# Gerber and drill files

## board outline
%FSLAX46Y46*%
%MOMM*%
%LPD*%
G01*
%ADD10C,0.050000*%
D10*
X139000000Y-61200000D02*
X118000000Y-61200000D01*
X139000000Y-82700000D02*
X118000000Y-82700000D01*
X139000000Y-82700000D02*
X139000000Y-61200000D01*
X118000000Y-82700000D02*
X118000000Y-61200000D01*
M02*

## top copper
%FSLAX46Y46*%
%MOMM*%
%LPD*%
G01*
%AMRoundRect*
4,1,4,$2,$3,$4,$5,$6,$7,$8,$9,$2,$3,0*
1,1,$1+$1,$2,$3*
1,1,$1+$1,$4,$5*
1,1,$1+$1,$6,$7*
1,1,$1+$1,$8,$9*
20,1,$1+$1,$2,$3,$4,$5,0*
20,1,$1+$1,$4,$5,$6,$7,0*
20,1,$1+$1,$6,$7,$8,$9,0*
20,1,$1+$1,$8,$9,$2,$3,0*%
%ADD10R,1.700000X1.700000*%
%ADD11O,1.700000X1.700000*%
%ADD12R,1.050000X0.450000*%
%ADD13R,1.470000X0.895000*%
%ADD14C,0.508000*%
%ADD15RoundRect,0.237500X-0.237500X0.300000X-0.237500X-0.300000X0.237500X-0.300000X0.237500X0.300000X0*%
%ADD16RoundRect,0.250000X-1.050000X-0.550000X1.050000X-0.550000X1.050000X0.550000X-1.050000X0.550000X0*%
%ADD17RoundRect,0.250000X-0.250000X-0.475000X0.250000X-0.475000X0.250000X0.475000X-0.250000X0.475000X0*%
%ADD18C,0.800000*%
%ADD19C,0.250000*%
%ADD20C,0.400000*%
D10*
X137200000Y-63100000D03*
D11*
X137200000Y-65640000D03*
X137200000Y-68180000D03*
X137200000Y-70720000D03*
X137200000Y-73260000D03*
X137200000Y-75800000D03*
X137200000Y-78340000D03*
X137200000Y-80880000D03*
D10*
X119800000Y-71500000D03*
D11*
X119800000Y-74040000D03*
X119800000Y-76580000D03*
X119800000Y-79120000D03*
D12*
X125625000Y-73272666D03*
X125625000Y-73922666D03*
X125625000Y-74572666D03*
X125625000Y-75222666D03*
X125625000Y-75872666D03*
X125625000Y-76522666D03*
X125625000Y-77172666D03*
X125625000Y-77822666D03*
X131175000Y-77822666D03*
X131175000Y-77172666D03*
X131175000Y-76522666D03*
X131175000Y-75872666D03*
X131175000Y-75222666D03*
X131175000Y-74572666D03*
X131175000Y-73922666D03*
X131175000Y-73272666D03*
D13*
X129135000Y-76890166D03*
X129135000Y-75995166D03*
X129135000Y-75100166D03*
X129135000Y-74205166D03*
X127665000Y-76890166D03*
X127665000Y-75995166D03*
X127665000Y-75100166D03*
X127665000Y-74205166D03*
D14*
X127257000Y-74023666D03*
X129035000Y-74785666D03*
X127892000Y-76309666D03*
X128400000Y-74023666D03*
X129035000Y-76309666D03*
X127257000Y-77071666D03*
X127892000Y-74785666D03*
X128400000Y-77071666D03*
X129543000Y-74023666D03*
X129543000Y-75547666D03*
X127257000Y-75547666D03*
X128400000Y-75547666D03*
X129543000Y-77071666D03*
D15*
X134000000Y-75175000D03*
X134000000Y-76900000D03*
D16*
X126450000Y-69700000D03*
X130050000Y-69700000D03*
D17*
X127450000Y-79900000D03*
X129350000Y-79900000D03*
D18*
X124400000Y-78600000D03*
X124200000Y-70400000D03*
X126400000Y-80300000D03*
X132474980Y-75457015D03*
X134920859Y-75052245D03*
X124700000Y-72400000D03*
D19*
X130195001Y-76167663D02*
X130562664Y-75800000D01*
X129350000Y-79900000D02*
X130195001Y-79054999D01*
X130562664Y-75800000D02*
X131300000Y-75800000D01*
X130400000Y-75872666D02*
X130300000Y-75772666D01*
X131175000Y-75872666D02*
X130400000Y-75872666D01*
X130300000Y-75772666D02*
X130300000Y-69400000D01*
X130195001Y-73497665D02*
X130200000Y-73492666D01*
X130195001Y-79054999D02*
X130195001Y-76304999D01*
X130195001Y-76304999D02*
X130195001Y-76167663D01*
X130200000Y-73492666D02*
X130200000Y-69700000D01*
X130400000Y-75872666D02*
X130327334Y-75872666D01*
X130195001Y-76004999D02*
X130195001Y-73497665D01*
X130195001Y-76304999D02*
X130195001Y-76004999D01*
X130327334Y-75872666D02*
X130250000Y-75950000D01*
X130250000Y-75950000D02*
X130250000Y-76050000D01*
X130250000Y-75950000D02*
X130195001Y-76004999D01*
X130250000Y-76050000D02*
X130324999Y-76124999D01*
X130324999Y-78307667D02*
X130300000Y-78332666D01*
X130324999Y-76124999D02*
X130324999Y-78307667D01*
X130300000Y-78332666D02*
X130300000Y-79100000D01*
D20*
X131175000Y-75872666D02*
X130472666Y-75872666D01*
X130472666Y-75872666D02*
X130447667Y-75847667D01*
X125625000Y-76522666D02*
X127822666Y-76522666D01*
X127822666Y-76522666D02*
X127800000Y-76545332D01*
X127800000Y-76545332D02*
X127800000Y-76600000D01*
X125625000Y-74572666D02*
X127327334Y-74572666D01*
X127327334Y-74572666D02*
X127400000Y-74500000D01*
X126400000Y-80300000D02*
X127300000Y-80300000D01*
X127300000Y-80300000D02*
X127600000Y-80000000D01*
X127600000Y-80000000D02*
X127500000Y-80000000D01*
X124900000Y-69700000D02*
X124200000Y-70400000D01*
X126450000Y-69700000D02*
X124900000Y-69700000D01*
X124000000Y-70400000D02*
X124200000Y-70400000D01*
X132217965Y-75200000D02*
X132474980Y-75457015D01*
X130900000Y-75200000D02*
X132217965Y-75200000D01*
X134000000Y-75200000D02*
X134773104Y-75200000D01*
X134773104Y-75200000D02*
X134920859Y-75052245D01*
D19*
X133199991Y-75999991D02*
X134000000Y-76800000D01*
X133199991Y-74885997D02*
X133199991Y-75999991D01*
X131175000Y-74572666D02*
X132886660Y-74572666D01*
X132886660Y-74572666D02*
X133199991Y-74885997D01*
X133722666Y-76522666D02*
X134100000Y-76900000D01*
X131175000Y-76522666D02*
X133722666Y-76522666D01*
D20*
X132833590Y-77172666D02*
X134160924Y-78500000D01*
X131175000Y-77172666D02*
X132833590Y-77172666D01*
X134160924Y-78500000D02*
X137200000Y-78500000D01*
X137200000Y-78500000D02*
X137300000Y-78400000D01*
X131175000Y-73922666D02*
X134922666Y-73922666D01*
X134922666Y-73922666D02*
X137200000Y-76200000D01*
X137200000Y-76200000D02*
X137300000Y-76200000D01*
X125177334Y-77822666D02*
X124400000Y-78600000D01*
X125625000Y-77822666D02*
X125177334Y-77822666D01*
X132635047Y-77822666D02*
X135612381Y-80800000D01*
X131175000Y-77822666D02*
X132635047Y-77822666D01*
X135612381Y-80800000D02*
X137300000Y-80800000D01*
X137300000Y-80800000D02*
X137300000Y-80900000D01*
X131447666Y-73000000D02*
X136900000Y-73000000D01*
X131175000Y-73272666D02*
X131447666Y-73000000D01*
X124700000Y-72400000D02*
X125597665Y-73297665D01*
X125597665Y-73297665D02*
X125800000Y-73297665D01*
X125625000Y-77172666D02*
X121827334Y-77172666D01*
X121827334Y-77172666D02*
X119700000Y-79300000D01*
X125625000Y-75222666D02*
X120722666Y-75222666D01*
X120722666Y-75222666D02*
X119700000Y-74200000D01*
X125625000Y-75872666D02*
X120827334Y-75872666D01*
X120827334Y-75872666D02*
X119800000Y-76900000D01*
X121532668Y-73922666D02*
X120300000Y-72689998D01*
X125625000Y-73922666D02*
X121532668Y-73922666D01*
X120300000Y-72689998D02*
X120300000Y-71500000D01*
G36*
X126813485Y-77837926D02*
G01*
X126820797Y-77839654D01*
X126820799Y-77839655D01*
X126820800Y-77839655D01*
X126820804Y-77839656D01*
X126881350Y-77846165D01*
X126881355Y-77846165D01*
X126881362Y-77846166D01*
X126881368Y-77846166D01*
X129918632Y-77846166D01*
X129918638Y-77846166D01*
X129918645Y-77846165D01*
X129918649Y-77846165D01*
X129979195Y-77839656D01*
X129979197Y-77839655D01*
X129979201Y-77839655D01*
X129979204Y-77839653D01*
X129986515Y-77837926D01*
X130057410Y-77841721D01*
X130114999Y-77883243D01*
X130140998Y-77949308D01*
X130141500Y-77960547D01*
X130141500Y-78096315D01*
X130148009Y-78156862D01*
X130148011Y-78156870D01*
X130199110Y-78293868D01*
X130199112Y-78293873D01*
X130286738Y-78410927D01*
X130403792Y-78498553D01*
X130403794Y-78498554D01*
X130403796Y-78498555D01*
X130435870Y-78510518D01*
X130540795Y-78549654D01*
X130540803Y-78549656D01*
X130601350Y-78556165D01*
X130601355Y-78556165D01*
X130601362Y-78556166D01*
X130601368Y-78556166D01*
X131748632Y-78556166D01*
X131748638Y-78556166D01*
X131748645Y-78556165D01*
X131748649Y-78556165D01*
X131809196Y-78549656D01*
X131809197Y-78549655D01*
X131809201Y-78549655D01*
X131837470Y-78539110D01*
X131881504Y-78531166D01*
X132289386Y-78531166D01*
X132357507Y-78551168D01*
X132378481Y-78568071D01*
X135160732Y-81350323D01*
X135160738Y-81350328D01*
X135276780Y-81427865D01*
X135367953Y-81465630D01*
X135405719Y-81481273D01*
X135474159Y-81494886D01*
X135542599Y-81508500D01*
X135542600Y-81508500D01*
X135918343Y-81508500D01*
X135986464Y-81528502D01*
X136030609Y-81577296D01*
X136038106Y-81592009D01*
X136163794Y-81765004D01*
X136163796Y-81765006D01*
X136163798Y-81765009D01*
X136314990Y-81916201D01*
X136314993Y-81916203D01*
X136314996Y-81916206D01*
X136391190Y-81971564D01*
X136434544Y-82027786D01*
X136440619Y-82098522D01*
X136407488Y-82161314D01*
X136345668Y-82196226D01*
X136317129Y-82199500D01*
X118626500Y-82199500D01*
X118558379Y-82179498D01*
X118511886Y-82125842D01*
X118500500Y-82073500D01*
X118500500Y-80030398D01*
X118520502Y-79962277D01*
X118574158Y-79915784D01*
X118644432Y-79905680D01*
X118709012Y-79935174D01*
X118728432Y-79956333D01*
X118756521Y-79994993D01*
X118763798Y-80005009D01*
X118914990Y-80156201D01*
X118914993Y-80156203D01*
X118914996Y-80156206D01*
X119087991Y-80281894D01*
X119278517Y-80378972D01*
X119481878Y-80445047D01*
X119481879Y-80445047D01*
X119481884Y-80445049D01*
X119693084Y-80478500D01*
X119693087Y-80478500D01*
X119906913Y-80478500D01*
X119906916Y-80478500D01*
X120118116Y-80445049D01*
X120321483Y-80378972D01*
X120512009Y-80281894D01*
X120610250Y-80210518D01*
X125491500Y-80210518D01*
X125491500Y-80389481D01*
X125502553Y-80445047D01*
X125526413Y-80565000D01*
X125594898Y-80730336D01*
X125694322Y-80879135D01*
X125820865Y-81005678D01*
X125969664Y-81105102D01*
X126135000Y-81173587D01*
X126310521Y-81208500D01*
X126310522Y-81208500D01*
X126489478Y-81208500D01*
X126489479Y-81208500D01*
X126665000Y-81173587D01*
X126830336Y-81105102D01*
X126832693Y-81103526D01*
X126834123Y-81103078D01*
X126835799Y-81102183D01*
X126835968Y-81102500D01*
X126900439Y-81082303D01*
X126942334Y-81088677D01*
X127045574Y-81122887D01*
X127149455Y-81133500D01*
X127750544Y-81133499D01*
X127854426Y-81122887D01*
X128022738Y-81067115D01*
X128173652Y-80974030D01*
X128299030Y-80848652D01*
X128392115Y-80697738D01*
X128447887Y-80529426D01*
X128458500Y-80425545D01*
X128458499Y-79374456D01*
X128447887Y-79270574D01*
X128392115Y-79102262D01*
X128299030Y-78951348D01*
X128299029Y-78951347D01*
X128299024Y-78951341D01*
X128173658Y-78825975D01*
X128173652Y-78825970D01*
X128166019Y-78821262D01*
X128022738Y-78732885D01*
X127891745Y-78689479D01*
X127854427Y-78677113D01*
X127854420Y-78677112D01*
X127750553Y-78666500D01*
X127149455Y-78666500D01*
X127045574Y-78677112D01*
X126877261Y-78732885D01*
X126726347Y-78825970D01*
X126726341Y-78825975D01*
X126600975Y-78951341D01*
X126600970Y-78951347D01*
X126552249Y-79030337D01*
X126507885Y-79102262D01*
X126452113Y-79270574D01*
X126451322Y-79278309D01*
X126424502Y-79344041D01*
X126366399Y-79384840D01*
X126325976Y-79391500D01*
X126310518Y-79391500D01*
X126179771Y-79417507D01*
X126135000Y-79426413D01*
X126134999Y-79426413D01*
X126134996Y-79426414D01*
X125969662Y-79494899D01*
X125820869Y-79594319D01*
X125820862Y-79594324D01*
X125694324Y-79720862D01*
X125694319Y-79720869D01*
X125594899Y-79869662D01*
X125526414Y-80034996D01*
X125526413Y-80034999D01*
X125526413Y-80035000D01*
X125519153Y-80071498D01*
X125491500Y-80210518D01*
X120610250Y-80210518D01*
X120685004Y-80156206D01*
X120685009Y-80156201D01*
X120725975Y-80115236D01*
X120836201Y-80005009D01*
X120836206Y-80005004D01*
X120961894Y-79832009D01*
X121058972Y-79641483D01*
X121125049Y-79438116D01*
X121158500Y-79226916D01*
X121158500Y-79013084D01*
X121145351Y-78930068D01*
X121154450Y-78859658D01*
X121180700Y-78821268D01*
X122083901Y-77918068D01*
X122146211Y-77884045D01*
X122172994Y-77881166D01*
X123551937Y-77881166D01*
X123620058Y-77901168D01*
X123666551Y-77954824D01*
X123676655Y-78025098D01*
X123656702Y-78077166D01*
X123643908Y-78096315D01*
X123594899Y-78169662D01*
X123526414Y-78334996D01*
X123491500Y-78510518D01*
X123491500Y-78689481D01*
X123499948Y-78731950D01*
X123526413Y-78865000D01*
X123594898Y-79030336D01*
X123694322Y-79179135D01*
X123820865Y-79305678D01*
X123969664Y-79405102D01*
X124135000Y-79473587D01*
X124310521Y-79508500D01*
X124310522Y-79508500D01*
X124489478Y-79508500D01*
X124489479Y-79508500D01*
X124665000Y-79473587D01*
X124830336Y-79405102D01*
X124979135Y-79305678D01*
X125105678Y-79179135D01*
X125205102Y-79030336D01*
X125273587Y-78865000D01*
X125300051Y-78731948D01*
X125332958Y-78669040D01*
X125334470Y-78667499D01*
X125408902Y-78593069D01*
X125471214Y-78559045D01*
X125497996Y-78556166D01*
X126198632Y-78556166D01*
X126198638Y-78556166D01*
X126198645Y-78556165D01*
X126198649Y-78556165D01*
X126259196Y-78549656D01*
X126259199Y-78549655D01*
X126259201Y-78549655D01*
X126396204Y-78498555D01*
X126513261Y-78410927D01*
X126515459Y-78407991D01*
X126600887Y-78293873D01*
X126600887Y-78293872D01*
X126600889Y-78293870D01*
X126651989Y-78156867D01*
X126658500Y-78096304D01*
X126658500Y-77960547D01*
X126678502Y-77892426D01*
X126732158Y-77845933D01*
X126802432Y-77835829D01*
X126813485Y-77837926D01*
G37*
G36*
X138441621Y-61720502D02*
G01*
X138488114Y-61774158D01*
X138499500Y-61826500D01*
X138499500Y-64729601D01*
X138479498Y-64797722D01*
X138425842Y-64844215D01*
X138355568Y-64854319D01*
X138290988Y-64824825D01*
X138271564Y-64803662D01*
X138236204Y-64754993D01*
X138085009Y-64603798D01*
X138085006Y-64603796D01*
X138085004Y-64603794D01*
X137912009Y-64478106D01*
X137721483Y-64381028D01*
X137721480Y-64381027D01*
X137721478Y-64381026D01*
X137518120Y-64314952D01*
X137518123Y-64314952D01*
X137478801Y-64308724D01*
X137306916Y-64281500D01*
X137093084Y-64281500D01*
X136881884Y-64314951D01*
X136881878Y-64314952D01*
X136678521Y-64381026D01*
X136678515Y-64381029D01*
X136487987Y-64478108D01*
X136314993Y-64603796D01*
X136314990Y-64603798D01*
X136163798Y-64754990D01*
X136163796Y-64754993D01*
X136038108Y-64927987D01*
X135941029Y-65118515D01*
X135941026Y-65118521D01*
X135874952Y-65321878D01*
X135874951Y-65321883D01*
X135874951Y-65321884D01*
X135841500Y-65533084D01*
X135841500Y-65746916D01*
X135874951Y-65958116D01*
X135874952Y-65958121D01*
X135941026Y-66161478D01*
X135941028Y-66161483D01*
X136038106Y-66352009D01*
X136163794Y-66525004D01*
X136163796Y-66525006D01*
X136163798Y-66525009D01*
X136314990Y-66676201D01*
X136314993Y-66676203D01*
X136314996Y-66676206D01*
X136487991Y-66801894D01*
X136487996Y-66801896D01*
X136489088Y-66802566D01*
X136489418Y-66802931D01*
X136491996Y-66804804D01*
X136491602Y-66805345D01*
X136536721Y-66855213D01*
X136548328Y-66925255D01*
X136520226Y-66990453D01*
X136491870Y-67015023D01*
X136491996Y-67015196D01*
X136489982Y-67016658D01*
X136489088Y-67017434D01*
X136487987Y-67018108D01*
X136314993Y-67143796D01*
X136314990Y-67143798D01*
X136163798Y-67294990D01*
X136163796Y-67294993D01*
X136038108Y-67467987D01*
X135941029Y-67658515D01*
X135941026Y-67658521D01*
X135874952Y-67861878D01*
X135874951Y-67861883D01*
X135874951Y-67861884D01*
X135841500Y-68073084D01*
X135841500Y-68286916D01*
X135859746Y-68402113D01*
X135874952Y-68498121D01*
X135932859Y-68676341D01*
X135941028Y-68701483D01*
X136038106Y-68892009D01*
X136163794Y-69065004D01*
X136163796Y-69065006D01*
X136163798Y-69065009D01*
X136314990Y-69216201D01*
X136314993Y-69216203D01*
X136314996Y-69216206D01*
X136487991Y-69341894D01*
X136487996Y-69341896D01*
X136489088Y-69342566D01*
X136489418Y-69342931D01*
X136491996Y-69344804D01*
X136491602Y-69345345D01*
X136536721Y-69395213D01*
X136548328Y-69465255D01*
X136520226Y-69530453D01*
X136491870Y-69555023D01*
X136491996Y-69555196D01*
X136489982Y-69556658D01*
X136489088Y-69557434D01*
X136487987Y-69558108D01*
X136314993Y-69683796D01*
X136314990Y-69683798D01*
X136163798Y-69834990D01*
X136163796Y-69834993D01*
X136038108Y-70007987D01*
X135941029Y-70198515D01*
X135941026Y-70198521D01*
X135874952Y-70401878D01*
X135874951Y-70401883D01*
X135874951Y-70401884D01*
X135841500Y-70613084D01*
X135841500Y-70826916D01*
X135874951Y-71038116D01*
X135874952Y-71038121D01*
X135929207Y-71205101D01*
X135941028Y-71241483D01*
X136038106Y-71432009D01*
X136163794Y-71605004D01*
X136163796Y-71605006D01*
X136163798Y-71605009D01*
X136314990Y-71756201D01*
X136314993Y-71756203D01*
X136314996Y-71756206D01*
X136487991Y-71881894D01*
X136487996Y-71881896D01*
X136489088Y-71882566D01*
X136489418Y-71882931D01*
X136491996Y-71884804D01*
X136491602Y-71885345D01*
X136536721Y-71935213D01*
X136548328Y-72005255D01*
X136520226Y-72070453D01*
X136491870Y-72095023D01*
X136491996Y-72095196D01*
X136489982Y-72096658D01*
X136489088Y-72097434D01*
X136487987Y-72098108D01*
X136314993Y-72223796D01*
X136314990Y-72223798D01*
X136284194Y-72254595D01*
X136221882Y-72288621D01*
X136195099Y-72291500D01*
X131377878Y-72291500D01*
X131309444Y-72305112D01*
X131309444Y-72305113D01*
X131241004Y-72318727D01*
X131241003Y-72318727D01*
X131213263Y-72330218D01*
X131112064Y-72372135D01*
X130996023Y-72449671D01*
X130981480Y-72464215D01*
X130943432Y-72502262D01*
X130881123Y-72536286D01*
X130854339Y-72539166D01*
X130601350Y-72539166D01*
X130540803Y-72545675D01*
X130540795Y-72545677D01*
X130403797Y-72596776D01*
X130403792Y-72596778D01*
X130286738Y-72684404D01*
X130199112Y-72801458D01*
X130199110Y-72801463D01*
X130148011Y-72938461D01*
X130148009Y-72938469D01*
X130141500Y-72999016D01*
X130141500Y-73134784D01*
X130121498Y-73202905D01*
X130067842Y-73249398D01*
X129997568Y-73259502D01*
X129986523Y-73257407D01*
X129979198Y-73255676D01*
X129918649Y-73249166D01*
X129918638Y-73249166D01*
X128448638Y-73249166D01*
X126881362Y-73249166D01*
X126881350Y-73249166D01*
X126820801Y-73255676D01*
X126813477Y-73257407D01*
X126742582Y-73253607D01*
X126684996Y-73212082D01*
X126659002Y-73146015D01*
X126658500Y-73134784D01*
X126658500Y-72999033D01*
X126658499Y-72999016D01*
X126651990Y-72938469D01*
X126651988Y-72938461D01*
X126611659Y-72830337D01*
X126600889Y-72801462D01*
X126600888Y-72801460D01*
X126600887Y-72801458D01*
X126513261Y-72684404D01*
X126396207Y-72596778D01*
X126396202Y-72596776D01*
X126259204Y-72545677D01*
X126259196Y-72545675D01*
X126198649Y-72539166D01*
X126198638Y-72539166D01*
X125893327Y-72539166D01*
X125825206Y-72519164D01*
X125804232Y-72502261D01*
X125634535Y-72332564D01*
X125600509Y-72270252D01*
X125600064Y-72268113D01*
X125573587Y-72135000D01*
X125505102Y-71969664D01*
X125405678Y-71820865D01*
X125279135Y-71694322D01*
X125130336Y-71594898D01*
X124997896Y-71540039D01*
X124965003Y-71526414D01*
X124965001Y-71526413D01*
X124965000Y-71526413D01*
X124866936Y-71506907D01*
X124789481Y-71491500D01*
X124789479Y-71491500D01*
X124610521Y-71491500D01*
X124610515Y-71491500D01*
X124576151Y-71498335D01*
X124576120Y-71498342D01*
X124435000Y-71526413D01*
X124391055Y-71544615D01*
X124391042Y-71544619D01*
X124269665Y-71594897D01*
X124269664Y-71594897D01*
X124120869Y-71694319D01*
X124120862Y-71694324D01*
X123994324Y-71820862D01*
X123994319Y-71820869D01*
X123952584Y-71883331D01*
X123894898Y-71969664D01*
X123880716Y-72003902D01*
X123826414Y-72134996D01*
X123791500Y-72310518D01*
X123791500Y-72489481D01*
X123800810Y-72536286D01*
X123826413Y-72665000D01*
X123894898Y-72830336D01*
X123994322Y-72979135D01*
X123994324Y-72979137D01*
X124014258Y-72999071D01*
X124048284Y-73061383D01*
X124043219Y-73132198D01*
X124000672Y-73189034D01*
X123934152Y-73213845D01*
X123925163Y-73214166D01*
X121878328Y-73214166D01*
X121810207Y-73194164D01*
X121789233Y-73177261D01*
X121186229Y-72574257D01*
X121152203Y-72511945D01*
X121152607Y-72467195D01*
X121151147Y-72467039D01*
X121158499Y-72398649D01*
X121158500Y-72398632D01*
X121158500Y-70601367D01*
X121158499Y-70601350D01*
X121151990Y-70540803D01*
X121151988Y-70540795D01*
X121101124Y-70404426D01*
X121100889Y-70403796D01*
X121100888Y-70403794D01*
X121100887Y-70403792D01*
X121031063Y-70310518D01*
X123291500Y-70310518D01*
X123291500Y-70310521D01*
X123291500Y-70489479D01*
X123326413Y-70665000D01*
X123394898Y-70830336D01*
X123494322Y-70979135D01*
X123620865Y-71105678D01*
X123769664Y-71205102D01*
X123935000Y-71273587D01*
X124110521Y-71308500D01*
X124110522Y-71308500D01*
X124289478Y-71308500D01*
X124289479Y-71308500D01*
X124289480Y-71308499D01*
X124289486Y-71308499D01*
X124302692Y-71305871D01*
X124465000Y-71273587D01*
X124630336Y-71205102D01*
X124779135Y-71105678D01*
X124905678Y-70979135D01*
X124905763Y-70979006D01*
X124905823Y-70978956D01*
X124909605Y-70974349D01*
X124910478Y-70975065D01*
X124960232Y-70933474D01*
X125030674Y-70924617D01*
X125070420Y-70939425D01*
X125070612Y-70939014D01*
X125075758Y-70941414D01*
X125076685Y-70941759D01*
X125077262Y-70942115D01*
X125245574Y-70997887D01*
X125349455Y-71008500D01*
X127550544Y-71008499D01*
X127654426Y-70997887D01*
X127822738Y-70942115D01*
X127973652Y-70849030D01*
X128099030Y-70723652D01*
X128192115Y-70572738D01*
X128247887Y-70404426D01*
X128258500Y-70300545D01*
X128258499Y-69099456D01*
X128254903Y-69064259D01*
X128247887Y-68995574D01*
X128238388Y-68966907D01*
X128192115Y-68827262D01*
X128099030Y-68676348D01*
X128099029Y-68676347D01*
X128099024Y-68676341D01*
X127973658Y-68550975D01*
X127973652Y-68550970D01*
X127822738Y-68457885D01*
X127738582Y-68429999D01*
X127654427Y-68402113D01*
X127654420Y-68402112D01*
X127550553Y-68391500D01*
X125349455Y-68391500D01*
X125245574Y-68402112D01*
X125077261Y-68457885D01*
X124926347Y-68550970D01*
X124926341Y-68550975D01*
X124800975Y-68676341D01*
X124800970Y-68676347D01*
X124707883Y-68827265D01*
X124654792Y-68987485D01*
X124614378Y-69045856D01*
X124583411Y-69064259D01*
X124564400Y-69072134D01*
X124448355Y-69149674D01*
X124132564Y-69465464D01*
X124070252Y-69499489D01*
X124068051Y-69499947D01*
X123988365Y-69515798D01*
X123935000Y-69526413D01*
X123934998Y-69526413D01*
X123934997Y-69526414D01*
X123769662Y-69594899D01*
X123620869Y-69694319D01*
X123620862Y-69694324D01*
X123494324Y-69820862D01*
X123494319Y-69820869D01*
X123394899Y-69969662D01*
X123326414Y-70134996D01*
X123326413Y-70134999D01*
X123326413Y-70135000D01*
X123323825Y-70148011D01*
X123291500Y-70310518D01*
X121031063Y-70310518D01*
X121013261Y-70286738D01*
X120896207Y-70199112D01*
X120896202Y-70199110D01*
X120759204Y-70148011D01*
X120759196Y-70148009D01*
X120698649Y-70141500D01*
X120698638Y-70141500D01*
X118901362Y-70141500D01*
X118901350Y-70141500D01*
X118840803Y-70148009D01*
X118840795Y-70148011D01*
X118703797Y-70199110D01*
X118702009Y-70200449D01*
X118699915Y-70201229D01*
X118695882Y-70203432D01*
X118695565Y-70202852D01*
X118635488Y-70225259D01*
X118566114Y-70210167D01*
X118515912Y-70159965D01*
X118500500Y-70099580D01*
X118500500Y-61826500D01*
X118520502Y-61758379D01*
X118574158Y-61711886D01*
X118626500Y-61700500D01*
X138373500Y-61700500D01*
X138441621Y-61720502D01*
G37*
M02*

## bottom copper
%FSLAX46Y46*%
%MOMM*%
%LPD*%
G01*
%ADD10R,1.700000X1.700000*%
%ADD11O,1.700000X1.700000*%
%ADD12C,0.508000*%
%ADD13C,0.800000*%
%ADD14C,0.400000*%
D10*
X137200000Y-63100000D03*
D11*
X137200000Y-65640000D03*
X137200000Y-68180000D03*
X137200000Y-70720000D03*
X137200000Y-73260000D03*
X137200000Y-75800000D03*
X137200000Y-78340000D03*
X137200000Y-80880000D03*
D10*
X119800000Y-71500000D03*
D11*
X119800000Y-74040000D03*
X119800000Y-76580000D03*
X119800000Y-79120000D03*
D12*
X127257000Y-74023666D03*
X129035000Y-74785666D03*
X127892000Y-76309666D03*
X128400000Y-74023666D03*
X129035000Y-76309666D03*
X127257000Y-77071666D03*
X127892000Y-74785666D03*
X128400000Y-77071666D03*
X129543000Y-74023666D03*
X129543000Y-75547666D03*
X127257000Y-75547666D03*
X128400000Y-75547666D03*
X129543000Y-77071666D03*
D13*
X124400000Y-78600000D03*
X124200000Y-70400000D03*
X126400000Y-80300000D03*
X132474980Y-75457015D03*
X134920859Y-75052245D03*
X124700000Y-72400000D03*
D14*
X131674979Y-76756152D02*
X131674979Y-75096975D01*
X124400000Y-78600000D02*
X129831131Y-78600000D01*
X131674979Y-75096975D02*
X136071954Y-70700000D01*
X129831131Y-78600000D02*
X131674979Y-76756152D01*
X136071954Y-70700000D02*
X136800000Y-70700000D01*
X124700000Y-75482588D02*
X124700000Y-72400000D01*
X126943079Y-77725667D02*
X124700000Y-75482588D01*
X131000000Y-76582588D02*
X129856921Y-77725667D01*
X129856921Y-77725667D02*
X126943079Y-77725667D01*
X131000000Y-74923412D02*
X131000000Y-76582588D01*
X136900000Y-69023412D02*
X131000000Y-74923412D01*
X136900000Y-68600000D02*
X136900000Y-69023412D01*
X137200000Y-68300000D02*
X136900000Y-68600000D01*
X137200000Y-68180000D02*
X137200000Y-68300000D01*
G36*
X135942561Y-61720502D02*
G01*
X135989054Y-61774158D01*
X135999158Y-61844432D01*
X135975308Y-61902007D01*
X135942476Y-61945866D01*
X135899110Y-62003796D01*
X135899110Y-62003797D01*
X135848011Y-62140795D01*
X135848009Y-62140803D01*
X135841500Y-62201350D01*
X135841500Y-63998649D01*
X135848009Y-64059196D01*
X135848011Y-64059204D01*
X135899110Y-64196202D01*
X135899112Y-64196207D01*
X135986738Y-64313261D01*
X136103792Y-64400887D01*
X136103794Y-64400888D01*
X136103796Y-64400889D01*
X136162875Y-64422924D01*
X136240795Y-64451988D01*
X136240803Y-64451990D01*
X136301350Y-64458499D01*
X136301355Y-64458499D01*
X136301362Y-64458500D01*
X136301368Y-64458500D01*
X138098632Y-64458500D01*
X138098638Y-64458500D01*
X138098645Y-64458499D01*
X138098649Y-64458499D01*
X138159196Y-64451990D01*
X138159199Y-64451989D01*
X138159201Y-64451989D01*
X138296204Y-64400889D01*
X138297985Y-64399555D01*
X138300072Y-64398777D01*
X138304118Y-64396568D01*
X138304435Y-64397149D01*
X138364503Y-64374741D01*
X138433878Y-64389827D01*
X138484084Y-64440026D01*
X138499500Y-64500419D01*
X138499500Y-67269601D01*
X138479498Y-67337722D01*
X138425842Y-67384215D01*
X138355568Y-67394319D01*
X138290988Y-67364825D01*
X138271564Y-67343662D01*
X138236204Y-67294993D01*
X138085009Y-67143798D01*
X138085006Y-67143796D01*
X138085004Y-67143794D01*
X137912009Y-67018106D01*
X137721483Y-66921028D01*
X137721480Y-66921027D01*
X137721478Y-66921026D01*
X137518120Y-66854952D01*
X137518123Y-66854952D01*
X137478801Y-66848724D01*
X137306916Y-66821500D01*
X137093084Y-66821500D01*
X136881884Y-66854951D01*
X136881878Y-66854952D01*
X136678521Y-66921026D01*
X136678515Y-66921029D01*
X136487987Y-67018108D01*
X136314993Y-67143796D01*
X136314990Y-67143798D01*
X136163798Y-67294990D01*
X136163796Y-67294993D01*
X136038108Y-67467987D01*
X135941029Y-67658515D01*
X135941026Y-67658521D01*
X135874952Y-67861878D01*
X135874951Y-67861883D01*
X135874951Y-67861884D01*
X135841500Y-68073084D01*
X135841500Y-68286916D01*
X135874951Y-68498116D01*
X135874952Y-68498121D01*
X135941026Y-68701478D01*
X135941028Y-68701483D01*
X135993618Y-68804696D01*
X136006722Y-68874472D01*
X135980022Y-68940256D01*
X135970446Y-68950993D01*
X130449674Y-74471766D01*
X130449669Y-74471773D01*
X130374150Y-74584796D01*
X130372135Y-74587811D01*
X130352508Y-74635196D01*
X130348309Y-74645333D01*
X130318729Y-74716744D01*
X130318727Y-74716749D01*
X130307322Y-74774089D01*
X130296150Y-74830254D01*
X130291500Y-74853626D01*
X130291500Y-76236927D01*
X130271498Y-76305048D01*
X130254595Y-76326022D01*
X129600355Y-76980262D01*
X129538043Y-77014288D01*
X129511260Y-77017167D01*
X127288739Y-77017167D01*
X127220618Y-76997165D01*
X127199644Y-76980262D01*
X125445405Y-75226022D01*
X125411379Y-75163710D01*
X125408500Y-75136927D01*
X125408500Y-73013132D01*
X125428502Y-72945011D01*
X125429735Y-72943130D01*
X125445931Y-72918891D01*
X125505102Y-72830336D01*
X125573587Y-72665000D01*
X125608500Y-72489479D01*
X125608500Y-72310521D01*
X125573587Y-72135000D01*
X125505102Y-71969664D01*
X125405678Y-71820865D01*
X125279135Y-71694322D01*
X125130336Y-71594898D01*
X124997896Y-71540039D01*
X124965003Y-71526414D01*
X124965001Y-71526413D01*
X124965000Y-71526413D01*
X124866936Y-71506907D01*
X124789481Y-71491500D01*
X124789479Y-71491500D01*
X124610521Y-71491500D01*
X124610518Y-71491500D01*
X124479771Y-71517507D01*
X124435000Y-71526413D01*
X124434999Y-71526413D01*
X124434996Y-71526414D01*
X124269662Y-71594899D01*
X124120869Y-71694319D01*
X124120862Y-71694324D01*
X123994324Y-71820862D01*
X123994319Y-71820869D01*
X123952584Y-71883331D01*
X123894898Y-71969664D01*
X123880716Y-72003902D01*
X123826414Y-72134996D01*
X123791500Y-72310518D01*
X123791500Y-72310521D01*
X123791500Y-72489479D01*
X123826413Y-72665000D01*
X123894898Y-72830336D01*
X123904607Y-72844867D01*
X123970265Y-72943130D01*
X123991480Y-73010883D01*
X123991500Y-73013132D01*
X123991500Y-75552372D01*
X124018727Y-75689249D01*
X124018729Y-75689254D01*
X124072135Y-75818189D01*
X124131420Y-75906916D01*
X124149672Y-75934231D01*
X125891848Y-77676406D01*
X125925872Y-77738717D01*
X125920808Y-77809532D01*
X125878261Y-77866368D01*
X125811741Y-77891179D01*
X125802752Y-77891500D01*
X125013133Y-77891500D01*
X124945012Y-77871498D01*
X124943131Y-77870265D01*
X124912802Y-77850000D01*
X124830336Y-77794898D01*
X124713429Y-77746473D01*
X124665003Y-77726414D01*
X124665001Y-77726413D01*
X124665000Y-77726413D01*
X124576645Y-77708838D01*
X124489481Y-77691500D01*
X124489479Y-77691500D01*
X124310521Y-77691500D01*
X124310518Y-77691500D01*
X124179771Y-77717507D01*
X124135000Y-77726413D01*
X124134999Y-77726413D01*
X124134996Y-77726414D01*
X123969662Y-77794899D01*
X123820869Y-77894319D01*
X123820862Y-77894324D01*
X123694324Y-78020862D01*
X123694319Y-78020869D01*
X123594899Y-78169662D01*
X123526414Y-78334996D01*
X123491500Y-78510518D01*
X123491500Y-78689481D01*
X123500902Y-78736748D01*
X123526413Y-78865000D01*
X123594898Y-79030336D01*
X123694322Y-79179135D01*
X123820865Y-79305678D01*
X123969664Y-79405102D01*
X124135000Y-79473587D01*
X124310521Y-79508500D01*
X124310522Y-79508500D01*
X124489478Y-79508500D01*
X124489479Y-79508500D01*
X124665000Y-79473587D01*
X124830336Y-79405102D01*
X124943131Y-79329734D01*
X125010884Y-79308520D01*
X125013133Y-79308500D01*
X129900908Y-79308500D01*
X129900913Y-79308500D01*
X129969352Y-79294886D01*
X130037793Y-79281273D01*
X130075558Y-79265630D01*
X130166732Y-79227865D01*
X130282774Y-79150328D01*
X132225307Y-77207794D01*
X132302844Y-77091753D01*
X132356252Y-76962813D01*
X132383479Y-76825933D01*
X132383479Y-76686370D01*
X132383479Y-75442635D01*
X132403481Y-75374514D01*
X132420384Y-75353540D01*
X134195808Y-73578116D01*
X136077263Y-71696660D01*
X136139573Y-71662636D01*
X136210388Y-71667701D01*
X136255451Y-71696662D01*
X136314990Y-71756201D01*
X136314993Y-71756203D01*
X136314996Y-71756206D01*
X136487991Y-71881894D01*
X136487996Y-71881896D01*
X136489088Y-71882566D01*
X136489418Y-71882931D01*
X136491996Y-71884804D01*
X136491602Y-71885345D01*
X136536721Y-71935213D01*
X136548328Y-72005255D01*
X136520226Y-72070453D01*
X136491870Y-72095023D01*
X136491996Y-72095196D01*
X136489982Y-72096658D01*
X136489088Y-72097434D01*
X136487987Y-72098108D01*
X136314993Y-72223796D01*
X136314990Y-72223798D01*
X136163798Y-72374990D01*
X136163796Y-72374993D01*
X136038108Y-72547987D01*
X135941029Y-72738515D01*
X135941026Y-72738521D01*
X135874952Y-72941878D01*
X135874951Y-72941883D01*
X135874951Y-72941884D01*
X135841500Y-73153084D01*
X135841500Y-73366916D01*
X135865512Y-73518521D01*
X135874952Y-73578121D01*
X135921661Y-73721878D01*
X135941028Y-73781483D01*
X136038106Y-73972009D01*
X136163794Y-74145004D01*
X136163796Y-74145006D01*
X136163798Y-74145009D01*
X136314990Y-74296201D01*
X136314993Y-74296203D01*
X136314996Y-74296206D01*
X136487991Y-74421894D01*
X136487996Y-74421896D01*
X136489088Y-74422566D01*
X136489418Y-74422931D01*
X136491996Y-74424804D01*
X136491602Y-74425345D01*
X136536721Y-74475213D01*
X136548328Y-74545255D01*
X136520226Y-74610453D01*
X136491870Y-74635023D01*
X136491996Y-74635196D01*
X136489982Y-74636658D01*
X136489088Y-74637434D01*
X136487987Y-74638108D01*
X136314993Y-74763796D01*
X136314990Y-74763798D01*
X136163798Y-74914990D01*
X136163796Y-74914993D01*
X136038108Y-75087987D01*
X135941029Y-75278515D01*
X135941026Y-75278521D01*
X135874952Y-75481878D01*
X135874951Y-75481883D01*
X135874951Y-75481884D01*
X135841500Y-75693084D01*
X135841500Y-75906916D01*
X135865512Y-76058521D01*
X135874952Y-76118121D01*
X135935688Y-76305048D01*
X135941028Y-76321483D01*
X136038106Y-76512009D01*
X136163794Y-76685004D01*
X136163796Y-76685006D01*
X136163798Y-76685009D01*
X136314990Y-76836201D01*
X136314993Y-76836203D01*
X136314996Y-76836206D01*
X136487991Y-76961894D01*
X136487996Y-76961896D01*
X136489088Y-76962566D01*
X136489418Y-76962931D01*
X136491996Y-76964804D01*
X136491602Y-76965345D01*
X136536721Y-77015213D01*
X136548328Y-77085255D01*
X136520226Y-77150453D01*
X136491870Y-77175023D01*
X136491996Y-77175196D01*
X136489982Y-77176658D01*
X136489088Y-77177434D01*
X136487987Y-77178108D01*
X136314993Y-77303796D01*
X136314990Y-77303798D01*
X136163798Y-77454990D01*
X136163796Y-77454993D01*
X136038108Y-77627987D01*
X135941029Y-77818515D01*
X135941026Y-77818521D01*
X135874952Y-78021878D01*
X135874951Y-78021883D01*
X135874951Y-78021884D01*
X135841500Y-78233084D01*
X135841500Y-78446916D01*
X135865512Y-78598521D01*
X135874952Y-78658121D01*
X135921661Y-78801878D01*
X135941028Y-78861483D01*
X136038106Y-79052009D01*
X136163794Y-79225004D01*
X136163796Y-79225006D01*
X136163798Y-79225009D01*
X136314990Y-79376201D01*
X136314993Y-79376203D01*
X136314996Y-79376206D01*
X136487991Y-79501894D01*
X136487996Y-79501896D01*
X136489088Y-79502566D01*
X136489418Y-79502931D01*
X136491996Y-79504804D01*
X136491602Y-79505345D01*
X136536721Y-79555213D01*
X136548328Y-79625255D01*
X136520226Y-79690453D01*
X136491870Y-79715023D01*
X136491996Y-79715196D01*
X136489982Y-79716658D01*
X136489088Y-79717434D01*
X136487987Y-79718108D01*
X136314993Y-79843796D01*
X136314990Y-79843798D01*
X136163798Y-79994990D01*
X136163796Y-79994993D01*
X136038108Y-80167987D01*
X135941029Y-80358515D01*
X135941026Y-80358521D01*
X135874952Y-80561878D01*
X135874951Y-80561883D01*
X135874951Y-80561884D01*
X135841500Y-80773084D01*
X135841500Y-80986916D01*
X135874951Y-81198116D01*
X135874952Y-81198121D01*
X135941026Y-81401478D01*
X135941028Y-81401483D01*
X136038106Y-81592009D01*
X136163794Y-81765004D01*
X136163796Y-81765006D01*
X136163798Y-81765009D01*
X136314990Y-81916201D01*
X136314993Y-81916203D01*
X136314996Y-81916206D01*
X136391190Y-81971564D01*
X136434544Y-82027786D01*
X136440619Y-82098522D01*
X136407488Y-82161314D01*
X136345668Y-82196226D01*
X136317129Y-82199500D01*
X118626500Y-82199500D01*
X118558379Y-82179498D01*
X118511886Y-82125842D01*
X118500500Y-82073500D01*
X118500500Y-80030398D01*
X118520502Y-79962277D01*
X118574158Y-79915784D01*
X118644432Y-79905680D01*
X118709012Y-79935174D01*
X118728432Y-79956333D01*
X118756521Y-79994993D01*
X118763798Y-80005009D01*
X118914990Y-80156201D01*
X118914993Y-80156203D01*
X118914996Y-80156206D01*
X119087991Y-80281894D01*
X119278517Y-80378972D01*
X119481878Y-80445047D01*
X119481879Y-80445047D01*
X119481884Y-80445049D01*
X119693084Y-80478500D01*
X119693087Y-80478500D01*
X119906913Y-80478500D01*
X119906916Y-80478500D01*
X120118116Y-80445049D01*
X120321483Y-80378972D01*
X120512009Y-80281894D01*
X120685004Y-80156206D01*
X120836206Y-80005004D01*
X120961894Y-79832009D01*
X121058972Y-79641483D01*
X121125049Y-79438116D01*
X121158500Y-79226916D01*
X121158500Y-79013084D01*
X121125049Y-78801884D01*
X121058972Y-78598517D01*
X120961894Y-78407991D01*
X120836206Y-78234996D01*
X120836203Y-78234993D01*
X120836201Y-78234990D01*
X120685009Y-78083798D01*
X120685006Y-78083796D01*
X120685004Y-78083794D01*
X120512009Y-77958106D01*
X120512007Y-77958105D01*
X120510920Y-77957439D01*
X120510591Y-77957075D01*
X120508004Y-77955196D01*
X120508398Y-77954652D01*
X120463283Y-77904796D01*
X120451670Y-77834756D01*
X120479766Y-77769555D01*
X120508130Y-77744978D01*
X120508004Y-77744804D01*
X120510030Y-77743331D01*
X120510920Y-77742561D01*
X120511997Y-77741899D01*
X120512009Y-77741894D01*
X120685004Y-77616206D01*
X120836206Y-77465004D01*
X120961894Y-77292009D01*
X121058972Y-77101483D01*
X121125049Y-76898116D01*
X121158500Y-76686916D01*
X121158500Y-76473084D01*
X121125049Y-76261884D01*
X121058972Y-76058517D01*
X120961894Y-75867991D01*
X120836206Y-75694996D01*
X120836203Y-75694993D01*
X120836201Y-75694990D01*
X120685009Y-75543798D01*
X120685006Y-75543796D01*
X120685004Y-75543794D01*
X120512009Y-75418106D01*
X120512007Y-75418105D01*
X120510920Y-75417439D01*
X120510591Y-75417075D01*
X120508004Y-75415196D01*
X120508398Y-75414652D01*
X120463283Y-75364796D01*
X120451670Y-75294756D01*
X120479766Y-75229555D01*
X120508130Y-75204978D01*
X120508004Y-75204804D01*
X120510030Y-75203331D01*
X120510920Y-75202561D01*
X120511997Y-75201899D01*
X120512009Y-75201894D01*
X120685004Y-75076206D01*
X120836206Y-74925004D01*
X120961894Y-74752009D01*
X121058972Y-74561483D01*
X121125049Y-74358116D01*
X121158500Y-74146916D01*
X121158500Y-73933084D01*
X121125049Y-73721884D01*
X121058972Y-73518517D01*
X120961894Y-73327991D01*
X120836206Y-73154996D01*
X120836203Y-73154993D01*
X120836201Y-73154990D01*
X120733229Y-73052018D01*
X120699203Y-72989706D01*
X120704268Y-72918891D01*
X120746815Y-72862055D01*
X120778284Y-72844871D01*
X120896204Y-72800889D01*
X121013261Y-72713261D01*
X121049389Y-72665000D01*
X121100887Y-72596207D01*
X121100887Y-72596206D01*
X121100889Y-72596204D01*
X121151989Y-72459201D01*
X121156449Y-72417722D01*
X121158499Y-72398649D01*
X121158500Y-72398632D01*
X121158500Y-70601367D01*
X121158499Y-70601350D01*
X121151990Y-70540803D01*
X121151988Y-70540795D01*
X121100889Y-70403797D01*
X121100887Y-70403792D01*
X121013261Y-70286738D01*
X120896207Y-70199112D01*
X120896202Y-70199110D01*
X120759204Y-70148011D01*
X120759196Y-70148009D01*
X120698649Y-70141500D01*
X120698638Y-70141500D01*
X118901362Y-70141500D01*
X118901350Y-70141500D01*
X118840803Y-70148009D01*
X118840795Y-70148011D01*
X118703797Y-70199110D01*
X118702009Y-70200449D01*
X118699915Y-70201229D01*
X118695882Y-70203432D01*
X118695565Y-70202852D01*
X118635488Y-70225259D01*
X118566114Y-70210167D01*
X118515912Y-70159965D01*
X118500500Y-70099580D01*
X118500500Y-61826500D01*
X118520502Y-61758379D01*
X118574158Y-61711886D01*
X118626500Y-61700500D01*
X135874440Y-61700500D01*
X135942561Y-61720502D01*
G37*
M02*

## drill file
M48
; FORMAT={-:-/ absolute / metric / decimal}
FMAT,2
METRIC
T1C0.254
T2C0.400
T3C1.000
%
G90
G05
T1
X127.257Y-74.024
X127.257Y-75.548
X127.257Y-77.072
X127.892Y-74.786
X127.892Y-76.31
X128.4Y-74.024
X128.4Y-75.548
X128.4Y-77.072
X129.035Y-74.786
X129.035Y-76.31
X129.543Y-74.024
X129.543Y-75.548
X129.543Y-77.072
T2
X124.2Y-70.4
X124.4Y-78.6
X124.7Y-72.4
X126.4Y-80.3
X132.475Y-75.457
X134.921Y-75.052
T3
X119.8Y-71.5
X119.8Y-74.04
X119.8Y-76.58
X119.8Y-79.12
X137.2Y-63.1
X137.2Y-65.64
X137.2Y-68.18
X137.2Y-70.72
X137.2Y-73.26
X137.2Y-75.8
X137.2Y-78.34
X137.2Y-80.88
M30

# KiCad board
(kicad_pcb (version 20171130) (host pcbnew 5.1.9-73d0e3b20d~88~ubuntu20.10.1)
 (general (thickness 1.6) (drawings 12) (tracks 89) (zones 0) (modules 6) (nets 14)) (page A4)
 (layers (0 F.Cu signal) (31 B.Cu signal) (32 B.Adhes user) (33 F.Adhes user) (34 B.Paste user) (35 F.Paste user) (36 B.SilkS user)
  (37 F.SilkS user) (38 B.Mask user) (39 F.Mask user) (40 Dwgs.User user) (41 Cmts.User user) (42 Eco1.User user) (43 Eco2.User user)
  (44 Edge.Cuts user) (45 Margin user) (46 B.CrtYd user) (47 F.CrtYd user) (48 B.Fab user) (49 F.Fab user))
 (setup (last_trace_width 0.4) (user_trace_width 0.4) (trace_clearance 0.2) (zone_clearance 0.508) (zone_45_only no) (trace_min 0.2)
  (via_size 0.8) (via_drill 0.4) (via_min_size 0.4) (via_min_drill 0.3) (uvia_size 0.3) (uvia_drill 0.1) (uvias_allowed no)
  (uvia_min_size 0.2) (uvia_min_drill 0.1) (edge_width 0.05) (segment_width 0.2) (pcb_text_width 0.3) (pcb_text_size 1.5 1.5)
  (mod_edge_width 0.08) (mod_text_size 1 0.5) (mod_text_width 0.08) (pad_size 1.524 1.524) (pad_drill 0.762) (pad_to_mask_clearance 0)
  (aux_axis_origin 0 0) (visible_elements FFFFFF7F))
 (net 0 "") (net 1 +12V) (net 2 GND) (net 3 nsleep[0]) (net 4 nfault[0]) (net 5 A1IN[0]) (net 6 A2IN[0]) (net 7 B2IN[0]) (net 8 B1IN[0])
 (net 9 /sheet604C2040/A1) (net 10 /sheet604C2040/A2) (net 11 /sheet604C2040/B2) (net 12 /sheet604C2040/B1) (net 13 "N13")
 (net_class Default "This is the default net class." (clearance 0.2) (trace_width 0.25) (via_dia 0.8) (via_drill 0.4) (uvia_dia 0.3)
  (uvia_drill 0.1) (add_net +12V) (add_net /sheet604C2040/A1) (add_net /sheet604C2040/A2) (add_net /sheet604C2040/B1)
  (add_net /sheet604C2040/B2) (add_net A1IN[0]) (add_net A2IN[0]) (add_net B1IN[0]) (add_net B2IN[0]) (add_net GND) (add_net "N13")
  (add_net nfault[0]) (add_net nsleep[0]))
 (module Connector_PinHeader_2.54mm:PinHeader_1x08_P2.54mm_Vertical (layer F.Cu) (at 137.2 63.1)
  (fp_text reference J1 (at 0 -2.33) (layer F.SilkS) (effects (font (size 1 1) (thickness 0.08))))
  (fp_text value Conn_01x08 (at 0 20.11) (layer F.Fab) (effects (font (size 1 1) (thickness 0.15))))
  (pad 1 thru_hole rect (at 0 0) (size 1.7 1.7) (drill 1) (layers *.Cu *.Mask) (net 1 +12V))
  (pad 2 thru_hole oval (at 0 2.54) (size 1.7 1.7) (drill 1) (layers *.Cu *.Mask) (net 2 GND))
  (pad 3 thru_hole oval (at 0 5.08) (size 1.7 1.7) (drill 1) (layers *.Cu *.Mask) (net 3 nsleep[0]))
  (pad 4 thru_hole oval (at 0 7.62) (size 1.7 1.7) (drill 1) (layers *.Cu *.Mask) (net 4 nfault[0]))
  (pad 5 thru_hole oval (at 0 10.16) (size 1.7 1.7) (drill 1) (layers *.Cu *.Mask) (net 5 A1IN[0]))
  (pad 6 thru_hole oval (at 0 12.7) (size 1.7 1.7) (drill 1) (layers *.Cu *.Mask) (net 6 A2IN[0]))
  (pad 7 thru_hole oval (at 0 15.24) (size 1.7 1.7) (drill 1) (layers *.Cu *.Mask) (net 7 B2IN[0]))
  (pad 8 thru_hole oval (at 0 17.78) (size 1.7 1.7) (drill 1) (layers *.Cu *.Mask) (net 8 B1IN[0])))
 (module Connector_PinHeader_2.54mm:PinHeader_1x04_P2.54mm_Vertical (layer F.Cu) (at 119.8 71.5)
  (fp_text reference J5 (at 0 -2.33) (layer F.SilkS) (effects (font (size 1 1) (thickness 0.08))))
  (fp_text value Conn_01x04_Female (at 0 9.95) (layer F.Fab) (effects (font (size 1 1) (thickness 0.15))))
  (pad 1 thru_hole rect (at 0 0) (size 1.7 1.7) (drill 1) (layers *.Cu *.Mask) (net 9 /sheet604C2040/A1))
  (pad 2 thru_hole oval (at 0 2.54) (size 1.7 1.7) (drill 1) (layers *.Cu *.Mask) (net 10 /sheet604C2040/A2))
  (pad 3 thru_hole oval (at 0 5.08) (size 1.7 1.7) (drill 1) (layers *.Cu *.Mask) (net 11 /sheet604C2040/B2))
  (pad 4 thru_hole oval (at 0 7.62) (size 1.7 1.7) (drill 1) (layers *.Cu *.Mask) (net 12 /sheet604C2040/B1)))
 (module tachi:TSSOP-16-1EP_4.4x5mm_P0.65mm (layer F.Cu) (at 128.4 75.547666)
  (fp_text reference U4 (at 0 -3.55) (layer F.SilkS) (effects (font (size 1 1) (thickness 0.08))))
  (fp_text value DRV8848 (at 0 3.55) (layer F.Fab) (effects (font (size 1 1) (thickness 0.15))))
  (pad 1 smd rect (at -2.775 -2.275) (size 1.05 0.45) (layers F.Cu F.Paste F.Mask) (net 3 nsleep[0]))
  (pad 2 smd rect (at -2.775 -1.625) (size 1.05 0.45) (layers F.Cu F.Paste F.Mask) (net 9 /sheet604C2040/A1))
  (pad 3 smd rect (at -2.775 -0.975) (size 1.05 0.45) (layers F.Cu F.Paste F.Mask) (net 2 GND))
  (pad 4 smd rect (at -2.775 -0.325) (size 1.05 0.45) (layers F.Cu F.Paste F.Mask) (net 10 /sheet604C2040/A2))
  (pad 5 smd rect (at -2.775 0.325) (size 1.05 0.45) (layers F.Cu F.Paste F.Mask) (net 11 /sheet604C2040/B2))
  (pad 6 smd rect (at -2.775 0.975) (size 1.05 0.45) (layers F.Cu F.Paste F.Mask) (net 2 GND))
  (pad 7 smd rect (at -2.775 1.625) (size 1.05 0.45) (layers F.Cu F.Paste F.Mask) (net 12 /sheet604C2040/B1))
  (pad 8 smd rect (at -2.775 2.275) (size 1.05 0.45) (layers F.Cu F.Paste F.Mask) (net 4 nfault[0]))
  (pad 9 smd rect (at 2.775 2.275) (size 1.05 0.45) (layers F.Cu F.Paste F.Mask) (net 8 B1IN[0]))
  (pad 10 smd rect (at 2.775 1.625) (size 1.05 0.45) (layers F.Cu F.Paste F.Mask) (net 7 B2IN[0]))
  (pad 11 smd rect (at 2.775 0.975) (size 1.05 0.45) (layers F.Cu F.Paste F.Mask) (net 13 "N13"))
  (pad 12 smd rect (at 2.775 0.325) (size 1.05 0.45) (layers F.Cu F.Paste F.Mask) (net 1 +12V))
  (pad 13 smd rect (at 2.775 -0.325) (size 1.05 0.45) (layers F.Cu F.Paste F.Mask) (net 2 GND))
  (pad 14 smd rect (at 2.775 -0.975) (size 1.05 0.45) (layers F.Cu F.Paste F.Mask) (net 13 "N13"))
  (pad 15 smd rect (at 2.775 -1.625) (size 1.05 0.45) (layers F.Cu F.Paste F.Mask) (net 6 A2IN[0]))
  (pad 16 smd rect (at 2.775 -2.275) (size 1.05 0.45) (layers F.Cu F.Paste F.Mask) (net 5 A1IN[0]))
  (pad 17 smd rect (at 0.735 1.3425) (size 1.47 0.895) (layers F.Cu F.Paste F.Mask) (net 2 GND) (solder_paste_margin_ratio -0.2))
  (pad 17 smd rect (at 0.735 0.4475) (size 1.47 0.895) (layers F.Cu F.Paste F.Mask) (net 2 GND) (solder_paste_margin_ratio -0.2))
  (pad 17 smd rect (at 0.735 -0.4475) (size 1.47 0.895) (layers F.Cu F.Paste F.Mask) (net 2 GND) (solder_paste_margin_ratio -0.2))
  (pad 17 smd rect (at 0.735 -1.3425) (size 1.47 0.895) (layers F.Cu F.Paste F.Mask) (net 2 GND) (solder_paste_margin_ratio -0.2))
  (pad 17 smd rect (at -0.735 1.3425) (size 1.47 0.895) (layers F.Cu F.Paste F.Mask) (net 2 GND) (solder_paste_margin_ratio -0.2))
  (pad 17 smd rect (at -0.735 0.4475) (size 1.47 0.895) (layers F.Cu F.Paste F.Mask) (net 2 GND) (solder_paste_margin_ratio -0.2))
  (pad 17 smd rect (at -0.735 -0.4475) (size 1.47 0.895) (layers F.Cu F.Paste F.Mask) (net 2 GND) (solder_paste_margin_ratio -0.2))
  (pad 17 smd rect (at -0.735 -1.3425) (size 1.47 0.895) (layers F.Cu F.Paste F.Mask) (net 2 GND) (solder_paste_margin_ratio -0.2))
  (pad 17 thru_hole circle (at -1.143 -1.524) (size 0.508 0.508) (drill 0.254) (layers *.Cu *.Mask) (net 2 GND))
  (pad 17 thru_hole circle (at 0.635 -0.762) (size 0.508 0.508) (drill 0.254) (layers *.Cu *.Mask) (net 2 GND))
  (pad 17 thru_hole circle (at -0.508 0.762) (size 0.508 0.508) (drill 0.254) (layers *.Cu *.Mask) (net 2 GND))
  (pad 17 thru_hole circle (at 0 -1.524) (size 0.508 0.508) (drill 0.254) (layers *.Cu *.Mask) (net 2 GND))
  (pad 17 thru_hole circle (at 0.635 0.762) (size 0.508 0.508) (drill 0.254) (layers *.Cu *.Mask) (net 2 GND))
  (pad 17 thru_hole circle (at -1.143 1.524) (size 0.508 0.508) (drill 0.254) (layers *.Cu *.Mask) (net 2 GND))
  (pad 17 thru_hole circle (at -0.508 -0.762) (size 0.508 0.508) (drill 0.254) (layers *.Cu *.Mask) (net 2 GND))
  (pad 17 thru_hole circle (at 0 1.524) (size 0.508 0.508) (drill 0.254) (layers *.Cu *.Mask) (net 2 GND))
  (pad 17 thru_hole circle (at 1.143 -1.524) (size 0.508 0.508) (drill 0.254) (layers *.Cu *.Mask) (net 2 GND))
  (pad 17 thru_hole circle (at 1.143 0) (size 0.508 0.508) (drill 0.254) (layers *.Cu *.Mask) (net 2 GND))
  (pad 17 thru_hole circle (at -1.143 0) (size 0.508 0.508) (drill 0.254) (layers *.Cu *.Mask) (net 2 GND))
  (pad 17 thru_hole circle (at 0 0) (size 0.508 0.508) (drill 0.254) (layers *.Cu *.Mask) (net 2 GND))
  (pad 17 thru_hole circle (at 1.143 1.524) (size 0.508 0.508) (drill 0.254) (layers *.Cu *.Mask) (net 2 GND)))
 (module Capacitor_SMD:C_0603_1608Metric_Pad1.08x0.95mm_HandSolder (layer F.Cu) (at 134 76.0375 270)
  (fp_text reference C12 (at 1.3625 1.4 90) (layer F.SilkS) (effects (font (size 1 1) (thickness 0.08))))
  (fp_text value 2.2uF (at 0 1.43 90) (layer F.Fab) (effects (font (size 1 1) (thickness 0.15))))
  (pad 1 smd roundrect (at -0.8625 0 270) (size 1.075 0.95) (layers F.Cu F.Paste F.Mask) (roundrect_rratio 0.25) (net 2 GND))
  (pad 2 smd roundrect (at 0.8625 0 270) (size 1.075 0.95) (layers F.Cu F.Paste F.Mask) (roundrect_rratio 0.25) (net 13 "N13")))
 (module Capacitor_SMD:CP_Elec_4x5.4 (layer F.Cu) (at 128.25 69.7)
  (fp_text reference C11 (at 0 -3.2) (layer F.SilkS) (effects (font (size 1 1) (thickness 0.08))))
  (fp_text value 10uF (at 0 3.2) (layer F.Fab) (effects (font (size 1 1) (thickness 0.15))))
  (pad 1 smd roundrect (at -1.8 0) (size 2.6 1.6) (layers F.Cu F.Paste F.Mask) (roundrect_rratio 0.15625) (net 2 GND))
  (pad 2 smd roundrect (at 1.8 0) (size 2.6 1.6) (layers F.Cu F.Paste F.Mask) (roundrect_rratio 0.15625) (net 1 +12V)))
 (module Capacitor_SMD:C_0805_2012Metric (layer F.Cu) (at 128.4 79.9)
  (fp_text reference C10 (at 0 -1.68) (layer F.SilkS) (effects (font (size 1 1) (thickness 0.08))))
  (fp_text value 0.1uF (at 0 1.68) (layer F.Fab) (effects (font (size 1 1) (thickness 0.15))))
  (pad 1 smd roundrect (at -0.95 0) (size 1 1.45) (layers F.Cu F.Paste F.Mask) (roundrect_rratio 0.25) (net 2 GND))
  (pad 2 smd roundrect (at 0.95 0) (size 1 1.45) (layers F.Cu F.Paste F.Mask) (roundrect_rratio 0.25) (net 1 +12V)))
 (gr_line (start 139 61.2) (end 118 61.2) (layer Edge.Cuts) (width 0.05))
 (gr_line (start 139 82.7) (end 118 82.7) (layer Edge.Cuts) (width 0.05))
 (gr_line (start 139 82.7) (end 139 61.2) (layer Edge.Cuts) (width 0.05))
 (gr_line (start 118 82.7) (end 118 61.2) (layer Edge.Cuts) (width 0.05))
 (via (at 124.4 78.6) (size 0.8) (drill 0.4) (layers F.Cu B.Cu) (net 4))
 (via (at 124.2 70.4) (size 0.8) (drill 0.4) (layers F.Cu B.Cu) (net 2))
 (segment (start 130.195001 76.167663) (end 130.562664 75.8) (width 0.25) (layer F.Cu) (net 1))
 (segment (start 129.35 79.9) (end 130.195001 79.054999) (width 0.25) (layer F.Cu) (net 1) (status 10))
 (segment (start 130.562664 75.8) (end 131.3 75.8) (width 0.25) (layer F.Cu) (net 1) (status 20))
 (segment (start 130.4 75.872666) (end 130.3 75.772666) (width 0.25) (layer F.Cu) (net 1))
 (segment (start 131.175 75.872666) (end 130.4 75.872666) (width 0.25) (layer F.Cu) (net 1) (status 10))
 (segment (start 130.3 75.772666) (end 130.3 69.4) (width 0.25) (layer F.Cu) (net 1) (status 20))
 (segment (start 130.195001 73.497665) (end 130.2 73.492666) (width 0.25) (layer F.Cu) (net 1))
 (segment (start 130.195001 79.054999) (end 130.195001 76.304999) (width 0.25) (layer F.Cu) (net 1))
 (segment (start 130.195001 76.304999) (end 130.195001 76.167663) (width 0.25) (layer F.Cu) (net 1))
 (segment (start 130.2 73.492666) (end 130.2 69.7) (width 0.25) (layer F.Cu) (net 1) (status 20))
 (segment (start 130.4 75.872666) (end 130.327334 75.872666) (width 0.25) (layer F.Cu) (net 1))
 (segment (start 130.195001 76.004999) (end 130.195001 73.497665) (width 0.25) (layer F.Cu) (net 1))
 (segment (start 130.195001 76.304999) (end 130.195001 76.004999) (width 0.25) (layer F.Cu) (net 1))
 (segment (start 130.327334 75.872666) (end 130.25 75.95) (width 0.25) (layer F.Cu) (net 1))
 (segment (start 130.25 75.95) (end 130.25 76.05) (width 0.25) (layer F.Cu) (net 1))
 (segment (start 130.25 75.95) (end 130.195001 76.004999) (width 0.25) (layer F.Cu) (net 1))
 (segment (start 130.25 76.05) (end 130.324999 76.124999) (width 0.25) (layer F.Cu) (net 1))
 (segment (start 130.324999 78.307667) (end 130.3 78.332666) (width 0.25) (layer F.Cu) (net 1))
 (segment (start 130.324999 76.124999) (end 130.324999 78.307667) (width 0.25) (layer F.Cu) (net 1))
 (segment (start 130.3 78.332666) (end 130.3 79.1) (width 0.25) (layer F.Cu) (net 1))
 (segment (start 131.175 75.872666) (end 130.472666 75.872666) (width 0.4) (layer F.Cu) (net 1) (status 10))
 (segment (start 130.472666 75.872666) (end 130.447667 75.847667) (width 0.4) (layer F.Cu) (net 1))
 (via (at 126.4 80.3) (size 0.8) (drill 0.4) (layers F.Cu B.Cu) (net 2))
 (segment (start 125.625 76.522666) (end 127.822666 76.522666) (width 0.4) (layer F.Cu) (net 2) (status 30))
 (segment (start 127.822666 76.522666) (end 127.8 76.545332) (width 0.4) (layer F.Cu) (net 2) (status 30))
 (segment (start 127.8 76.545332) (end 127.8 76.6) (width 0.4) (layer F.Cu) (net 2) (status 30))
 (segment (start 125.625 74.572666) (end 127.327334 74.572666) (width 0.4) (layer F.Cu) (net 2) (status 30))
 (segment (start 127.327334 74.572666) (end 127.4 74.5) (width 0.4) (layer F.Cu) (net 2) (status 30))
 (segment (start 126.4 80.3) (end 127.3 80.3) (width 0.4) (layer F.Cu) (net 2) (status 20))
 (segment (start 127.3 80.3) (end 127.6 80) (width 0.4) (layer F.Cu) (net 2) (status 30))
 (segment (start 127.6 80) (end 127.5 80) (width 0.4) (layer F.Cu) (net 2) (status 30))
 (segment (start 124.9 69.7) (end 124.2 70.4) (width 0.4) (layer F.Cu) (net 2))
 (segment (start 126.45 69.7) (end 124.9 69.7) (width 0.4) (layer F.Cu) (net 2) (status 10))
 (segment (start 124 70.4) (end 124.2 70.4) (width 0.4) (layer F.Cu) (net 2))
 (segment (start 132.217965 75.2) (end 132.47498 75.457015) (width 0.4) (layer F.Cu) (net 2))
 (via (at 132.47498 75.457015) (size 0.8) (drill 0.4) (layers F.Cu B.Cu) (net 2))
 (segment (start 130.9 75.2) (end 132.217965 75.2) (width 0.4) (layer F.Cu) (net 2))
 (via (at 134.920859 75.052245) (size 0.8) (drill 0.4) (layers F.Cu B.Cu) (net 2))
 (segment (start 134 75.2) (end 134.773104 75.2) (width 0.4) (layer F.Cu) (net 2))
 (segment (start 134.773104 75.2) (end 134.920859 75.052245) (width 0.4) (layer F.Cu) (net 2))
 (segment (start 133.199991 75.999991) (end 134 76.8) (width 0.25) (layer F.Cu) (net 13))
 (segment (start 133.199991 74.885997) (end 133.199991 75.999991) (width 0.25) (layer F.Cu) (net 13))
 (segment (start 131.175 74.572666) (end 132.88666 74.572666) (width 0.25) (layer F.Cu) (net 13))
 (segment (start 132.88666 74.572666) (end 133.199991 74.885997) (width 0.25) (layer F.Cu) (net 13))
 (segment (start 133.722666 76.522666) (end 134.1 76.9) (width 0.25) (layer F.Cu) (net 13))
 (segment (start 131.175 76.522666) (end 133.722666 76.522666) (width 0.25) (layer F.Cu) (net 13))
 (segment (start 132.83359 77.172666) (end 134.160924 78.5) (width 0.4) (layer F.Cu) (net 7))
 (segment (start 131.175 77.172666) (end 132.83359 77.172666) (width 0.4) (layer F.Cu) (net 7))
 (segment (start 134.160924 78.5) (end 137.2 78.5) (width 0.4) (layer F.Cu) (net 7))
 (segment (start 137.2 78.5) (end 137.3 78.4) (width 0.4) (layer F.Cu) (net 7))
 (segment (start 131.175 73.922666) (end 134.922666 73.922666) (width 0.4) (layer F.Cu) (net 6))
 (segment (start 134.922666 73.922666) (end 137.2 76.2) (width 0.4) (layer F.Cu) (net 6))
 (segment (start 137.2 76.2) (end 137.3 76.2) (width 0.4) (layer F.Cu) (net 6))
 (via (at 124.7 72.4) (size 0.8) (drill 0.4) (layers F.Cu B.Cu) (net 3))
 (segment (start 125.177334 77.822666) (end 124.4 78.6) (width 0.4) (layer F.Cu) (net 4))
 (segment (start 125.625 77.822666) (end 125.177334 77.822666) (width 0.4) (layer F.Cu) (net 4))
 (segment (start 131.674979 76.756152) (end 131.674979 75.096975) (width 0.4) (layer B.Cu) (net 4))
 (segment (start 124.4 78.6) (end 129.831131 78.6) (width 0.4) (layer B.Cu) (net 4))
 (segment (start 131.674979 75.096975) (end 136.071954 70.7) (width 0.4) (layer B.Cu) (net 4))
 (segment (start 129.831131 78.6) (end 131.674979 76.756152) (width 0.4) (layer B.Cu) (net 4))
 (segment (start 136.071954 70.7) (end 136.8 70.7) (width 0.4) (layer B.Cu) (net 4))
 (segment (start 132.635047 77.822666) (end 135.612381 80.8) (width 0.4) (layer F.Cu) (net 8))
 (segment (start 131.175 77.822666) (end 132.635047 77.822666) (width 0.4) (layer F.Cu) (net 8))
 (segment (start 135.612381 80.8) (end 137.3 80.8) (width 0.4) (layer F.Cu) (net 8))
 (segment (start 137.3 80.8) (end 137.3 80.9) (width 0.4) (layer F.Cu) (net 8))
 (segment (start 131.447666 73) (end 136.9 73) (width 0.4) (layer F.Cu) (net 5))
 (segment (start 131.175 73.272666) (end 131.447666 73) (width 0.4) (layer F.Cu) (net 5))
 (segment (start 124.7 72.4) (end 125.597665 73.297665) (width 0.4) (layer F.Cu) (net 3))
 (segment (start 125.597665 73.297665) (end 125.8 73.297665) (width 0.4) (layer F.Cu) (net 3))
 (segment (start 124.7 75.482588) (end 124.7 72.4) (width 0.4) (layer B.Cu) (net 3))
 (segment (start 126.943079 77.725667) (end 124.7 75.482588) (width 0.4) (layer B.Cu) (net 3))
 (segment (start 131 76.582588) (end 129.856921 77.725667) (width 0.4) (layer B.Cu) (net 3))
 (segment (start 129.856921 77.725667) (end 126.943079 77.725667) (width 0.4) (layer B.Cu) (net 3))
 (segment (start 131 74.923412) (end 131 76.582588) (width 0.4) (layer B.Cu) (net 3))
 (segment (start 136.9 69.023412) (end 131 74.923412) (width 0.4) (layer B.Cu) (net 3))
 (segment (start 136.9 68.6) (end 136.9 69.023412) (width 0.4) (layer B.Cu) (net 3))
 (segment (start 137.2 68.3) (end 136.9 68.6) (width 0.4) (layer B.Cu) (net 3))
 (segment (start 137.2 68.18) (end 137.2 68.3) (width 0.4) (layer B.Cu) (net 3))
 (segment (start 125.625 77.172666) (end 121.827334 77.172666) (width 0.4) (layer F.Cu) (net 12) (status 10))
 (segment (start 121.827334 77.172666) (end 119.7 79.3) (width 0.4) (layer F.Cu) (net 12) (status 20))
 (segment (start 125.625 75.222666) (end 120.722666 75.222666) (width 0.4) (layer F.Cu) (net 10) (status 10))
 (segment (start 120.722666 75.222666) (end 119.7 74.2) (width 0.4) (layer F.Cu) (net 10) (status 20))
 (segment (start 125.625 75.872666) (end 120.827334 75.872666) (width 0.4) (layer F.Cu) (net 11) (status 10))
 (segment (start 120.827334 75.872666) (end 119.8 76.9) (width 0.4) (layer F.Cu) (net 11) (status 20))
 (segment (start 121.532668 73.922666) (end 120.3 72.689998) (width 0.4) (layer F.Cu) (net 9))
 (segment (start 125.625 73.922666) (end 121.532668 73.922666) (width 0.4) (layer F.Cu) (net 9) (status 10))
 (segment (start 120.3 72.689998) (end 120.3 71.5) (width 0.4) (layer F.Cu) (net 9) (status 20))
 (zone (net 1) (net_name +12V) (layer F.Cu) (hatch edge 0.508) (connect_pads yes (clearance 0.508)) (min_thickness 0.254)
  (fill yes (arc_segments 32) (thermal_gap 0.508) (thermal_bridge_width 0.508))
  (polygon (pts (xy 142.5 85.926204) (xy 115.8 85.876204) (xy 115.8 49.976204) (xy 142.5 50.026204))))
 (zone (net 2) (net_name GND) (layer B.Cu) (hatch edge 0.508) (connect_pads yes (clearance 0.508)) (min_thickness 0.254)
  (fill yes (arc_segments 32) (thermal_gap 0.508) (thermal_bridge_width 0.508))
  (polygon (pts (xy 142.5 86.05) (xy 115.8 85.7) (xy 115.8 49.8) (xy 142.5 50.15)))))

